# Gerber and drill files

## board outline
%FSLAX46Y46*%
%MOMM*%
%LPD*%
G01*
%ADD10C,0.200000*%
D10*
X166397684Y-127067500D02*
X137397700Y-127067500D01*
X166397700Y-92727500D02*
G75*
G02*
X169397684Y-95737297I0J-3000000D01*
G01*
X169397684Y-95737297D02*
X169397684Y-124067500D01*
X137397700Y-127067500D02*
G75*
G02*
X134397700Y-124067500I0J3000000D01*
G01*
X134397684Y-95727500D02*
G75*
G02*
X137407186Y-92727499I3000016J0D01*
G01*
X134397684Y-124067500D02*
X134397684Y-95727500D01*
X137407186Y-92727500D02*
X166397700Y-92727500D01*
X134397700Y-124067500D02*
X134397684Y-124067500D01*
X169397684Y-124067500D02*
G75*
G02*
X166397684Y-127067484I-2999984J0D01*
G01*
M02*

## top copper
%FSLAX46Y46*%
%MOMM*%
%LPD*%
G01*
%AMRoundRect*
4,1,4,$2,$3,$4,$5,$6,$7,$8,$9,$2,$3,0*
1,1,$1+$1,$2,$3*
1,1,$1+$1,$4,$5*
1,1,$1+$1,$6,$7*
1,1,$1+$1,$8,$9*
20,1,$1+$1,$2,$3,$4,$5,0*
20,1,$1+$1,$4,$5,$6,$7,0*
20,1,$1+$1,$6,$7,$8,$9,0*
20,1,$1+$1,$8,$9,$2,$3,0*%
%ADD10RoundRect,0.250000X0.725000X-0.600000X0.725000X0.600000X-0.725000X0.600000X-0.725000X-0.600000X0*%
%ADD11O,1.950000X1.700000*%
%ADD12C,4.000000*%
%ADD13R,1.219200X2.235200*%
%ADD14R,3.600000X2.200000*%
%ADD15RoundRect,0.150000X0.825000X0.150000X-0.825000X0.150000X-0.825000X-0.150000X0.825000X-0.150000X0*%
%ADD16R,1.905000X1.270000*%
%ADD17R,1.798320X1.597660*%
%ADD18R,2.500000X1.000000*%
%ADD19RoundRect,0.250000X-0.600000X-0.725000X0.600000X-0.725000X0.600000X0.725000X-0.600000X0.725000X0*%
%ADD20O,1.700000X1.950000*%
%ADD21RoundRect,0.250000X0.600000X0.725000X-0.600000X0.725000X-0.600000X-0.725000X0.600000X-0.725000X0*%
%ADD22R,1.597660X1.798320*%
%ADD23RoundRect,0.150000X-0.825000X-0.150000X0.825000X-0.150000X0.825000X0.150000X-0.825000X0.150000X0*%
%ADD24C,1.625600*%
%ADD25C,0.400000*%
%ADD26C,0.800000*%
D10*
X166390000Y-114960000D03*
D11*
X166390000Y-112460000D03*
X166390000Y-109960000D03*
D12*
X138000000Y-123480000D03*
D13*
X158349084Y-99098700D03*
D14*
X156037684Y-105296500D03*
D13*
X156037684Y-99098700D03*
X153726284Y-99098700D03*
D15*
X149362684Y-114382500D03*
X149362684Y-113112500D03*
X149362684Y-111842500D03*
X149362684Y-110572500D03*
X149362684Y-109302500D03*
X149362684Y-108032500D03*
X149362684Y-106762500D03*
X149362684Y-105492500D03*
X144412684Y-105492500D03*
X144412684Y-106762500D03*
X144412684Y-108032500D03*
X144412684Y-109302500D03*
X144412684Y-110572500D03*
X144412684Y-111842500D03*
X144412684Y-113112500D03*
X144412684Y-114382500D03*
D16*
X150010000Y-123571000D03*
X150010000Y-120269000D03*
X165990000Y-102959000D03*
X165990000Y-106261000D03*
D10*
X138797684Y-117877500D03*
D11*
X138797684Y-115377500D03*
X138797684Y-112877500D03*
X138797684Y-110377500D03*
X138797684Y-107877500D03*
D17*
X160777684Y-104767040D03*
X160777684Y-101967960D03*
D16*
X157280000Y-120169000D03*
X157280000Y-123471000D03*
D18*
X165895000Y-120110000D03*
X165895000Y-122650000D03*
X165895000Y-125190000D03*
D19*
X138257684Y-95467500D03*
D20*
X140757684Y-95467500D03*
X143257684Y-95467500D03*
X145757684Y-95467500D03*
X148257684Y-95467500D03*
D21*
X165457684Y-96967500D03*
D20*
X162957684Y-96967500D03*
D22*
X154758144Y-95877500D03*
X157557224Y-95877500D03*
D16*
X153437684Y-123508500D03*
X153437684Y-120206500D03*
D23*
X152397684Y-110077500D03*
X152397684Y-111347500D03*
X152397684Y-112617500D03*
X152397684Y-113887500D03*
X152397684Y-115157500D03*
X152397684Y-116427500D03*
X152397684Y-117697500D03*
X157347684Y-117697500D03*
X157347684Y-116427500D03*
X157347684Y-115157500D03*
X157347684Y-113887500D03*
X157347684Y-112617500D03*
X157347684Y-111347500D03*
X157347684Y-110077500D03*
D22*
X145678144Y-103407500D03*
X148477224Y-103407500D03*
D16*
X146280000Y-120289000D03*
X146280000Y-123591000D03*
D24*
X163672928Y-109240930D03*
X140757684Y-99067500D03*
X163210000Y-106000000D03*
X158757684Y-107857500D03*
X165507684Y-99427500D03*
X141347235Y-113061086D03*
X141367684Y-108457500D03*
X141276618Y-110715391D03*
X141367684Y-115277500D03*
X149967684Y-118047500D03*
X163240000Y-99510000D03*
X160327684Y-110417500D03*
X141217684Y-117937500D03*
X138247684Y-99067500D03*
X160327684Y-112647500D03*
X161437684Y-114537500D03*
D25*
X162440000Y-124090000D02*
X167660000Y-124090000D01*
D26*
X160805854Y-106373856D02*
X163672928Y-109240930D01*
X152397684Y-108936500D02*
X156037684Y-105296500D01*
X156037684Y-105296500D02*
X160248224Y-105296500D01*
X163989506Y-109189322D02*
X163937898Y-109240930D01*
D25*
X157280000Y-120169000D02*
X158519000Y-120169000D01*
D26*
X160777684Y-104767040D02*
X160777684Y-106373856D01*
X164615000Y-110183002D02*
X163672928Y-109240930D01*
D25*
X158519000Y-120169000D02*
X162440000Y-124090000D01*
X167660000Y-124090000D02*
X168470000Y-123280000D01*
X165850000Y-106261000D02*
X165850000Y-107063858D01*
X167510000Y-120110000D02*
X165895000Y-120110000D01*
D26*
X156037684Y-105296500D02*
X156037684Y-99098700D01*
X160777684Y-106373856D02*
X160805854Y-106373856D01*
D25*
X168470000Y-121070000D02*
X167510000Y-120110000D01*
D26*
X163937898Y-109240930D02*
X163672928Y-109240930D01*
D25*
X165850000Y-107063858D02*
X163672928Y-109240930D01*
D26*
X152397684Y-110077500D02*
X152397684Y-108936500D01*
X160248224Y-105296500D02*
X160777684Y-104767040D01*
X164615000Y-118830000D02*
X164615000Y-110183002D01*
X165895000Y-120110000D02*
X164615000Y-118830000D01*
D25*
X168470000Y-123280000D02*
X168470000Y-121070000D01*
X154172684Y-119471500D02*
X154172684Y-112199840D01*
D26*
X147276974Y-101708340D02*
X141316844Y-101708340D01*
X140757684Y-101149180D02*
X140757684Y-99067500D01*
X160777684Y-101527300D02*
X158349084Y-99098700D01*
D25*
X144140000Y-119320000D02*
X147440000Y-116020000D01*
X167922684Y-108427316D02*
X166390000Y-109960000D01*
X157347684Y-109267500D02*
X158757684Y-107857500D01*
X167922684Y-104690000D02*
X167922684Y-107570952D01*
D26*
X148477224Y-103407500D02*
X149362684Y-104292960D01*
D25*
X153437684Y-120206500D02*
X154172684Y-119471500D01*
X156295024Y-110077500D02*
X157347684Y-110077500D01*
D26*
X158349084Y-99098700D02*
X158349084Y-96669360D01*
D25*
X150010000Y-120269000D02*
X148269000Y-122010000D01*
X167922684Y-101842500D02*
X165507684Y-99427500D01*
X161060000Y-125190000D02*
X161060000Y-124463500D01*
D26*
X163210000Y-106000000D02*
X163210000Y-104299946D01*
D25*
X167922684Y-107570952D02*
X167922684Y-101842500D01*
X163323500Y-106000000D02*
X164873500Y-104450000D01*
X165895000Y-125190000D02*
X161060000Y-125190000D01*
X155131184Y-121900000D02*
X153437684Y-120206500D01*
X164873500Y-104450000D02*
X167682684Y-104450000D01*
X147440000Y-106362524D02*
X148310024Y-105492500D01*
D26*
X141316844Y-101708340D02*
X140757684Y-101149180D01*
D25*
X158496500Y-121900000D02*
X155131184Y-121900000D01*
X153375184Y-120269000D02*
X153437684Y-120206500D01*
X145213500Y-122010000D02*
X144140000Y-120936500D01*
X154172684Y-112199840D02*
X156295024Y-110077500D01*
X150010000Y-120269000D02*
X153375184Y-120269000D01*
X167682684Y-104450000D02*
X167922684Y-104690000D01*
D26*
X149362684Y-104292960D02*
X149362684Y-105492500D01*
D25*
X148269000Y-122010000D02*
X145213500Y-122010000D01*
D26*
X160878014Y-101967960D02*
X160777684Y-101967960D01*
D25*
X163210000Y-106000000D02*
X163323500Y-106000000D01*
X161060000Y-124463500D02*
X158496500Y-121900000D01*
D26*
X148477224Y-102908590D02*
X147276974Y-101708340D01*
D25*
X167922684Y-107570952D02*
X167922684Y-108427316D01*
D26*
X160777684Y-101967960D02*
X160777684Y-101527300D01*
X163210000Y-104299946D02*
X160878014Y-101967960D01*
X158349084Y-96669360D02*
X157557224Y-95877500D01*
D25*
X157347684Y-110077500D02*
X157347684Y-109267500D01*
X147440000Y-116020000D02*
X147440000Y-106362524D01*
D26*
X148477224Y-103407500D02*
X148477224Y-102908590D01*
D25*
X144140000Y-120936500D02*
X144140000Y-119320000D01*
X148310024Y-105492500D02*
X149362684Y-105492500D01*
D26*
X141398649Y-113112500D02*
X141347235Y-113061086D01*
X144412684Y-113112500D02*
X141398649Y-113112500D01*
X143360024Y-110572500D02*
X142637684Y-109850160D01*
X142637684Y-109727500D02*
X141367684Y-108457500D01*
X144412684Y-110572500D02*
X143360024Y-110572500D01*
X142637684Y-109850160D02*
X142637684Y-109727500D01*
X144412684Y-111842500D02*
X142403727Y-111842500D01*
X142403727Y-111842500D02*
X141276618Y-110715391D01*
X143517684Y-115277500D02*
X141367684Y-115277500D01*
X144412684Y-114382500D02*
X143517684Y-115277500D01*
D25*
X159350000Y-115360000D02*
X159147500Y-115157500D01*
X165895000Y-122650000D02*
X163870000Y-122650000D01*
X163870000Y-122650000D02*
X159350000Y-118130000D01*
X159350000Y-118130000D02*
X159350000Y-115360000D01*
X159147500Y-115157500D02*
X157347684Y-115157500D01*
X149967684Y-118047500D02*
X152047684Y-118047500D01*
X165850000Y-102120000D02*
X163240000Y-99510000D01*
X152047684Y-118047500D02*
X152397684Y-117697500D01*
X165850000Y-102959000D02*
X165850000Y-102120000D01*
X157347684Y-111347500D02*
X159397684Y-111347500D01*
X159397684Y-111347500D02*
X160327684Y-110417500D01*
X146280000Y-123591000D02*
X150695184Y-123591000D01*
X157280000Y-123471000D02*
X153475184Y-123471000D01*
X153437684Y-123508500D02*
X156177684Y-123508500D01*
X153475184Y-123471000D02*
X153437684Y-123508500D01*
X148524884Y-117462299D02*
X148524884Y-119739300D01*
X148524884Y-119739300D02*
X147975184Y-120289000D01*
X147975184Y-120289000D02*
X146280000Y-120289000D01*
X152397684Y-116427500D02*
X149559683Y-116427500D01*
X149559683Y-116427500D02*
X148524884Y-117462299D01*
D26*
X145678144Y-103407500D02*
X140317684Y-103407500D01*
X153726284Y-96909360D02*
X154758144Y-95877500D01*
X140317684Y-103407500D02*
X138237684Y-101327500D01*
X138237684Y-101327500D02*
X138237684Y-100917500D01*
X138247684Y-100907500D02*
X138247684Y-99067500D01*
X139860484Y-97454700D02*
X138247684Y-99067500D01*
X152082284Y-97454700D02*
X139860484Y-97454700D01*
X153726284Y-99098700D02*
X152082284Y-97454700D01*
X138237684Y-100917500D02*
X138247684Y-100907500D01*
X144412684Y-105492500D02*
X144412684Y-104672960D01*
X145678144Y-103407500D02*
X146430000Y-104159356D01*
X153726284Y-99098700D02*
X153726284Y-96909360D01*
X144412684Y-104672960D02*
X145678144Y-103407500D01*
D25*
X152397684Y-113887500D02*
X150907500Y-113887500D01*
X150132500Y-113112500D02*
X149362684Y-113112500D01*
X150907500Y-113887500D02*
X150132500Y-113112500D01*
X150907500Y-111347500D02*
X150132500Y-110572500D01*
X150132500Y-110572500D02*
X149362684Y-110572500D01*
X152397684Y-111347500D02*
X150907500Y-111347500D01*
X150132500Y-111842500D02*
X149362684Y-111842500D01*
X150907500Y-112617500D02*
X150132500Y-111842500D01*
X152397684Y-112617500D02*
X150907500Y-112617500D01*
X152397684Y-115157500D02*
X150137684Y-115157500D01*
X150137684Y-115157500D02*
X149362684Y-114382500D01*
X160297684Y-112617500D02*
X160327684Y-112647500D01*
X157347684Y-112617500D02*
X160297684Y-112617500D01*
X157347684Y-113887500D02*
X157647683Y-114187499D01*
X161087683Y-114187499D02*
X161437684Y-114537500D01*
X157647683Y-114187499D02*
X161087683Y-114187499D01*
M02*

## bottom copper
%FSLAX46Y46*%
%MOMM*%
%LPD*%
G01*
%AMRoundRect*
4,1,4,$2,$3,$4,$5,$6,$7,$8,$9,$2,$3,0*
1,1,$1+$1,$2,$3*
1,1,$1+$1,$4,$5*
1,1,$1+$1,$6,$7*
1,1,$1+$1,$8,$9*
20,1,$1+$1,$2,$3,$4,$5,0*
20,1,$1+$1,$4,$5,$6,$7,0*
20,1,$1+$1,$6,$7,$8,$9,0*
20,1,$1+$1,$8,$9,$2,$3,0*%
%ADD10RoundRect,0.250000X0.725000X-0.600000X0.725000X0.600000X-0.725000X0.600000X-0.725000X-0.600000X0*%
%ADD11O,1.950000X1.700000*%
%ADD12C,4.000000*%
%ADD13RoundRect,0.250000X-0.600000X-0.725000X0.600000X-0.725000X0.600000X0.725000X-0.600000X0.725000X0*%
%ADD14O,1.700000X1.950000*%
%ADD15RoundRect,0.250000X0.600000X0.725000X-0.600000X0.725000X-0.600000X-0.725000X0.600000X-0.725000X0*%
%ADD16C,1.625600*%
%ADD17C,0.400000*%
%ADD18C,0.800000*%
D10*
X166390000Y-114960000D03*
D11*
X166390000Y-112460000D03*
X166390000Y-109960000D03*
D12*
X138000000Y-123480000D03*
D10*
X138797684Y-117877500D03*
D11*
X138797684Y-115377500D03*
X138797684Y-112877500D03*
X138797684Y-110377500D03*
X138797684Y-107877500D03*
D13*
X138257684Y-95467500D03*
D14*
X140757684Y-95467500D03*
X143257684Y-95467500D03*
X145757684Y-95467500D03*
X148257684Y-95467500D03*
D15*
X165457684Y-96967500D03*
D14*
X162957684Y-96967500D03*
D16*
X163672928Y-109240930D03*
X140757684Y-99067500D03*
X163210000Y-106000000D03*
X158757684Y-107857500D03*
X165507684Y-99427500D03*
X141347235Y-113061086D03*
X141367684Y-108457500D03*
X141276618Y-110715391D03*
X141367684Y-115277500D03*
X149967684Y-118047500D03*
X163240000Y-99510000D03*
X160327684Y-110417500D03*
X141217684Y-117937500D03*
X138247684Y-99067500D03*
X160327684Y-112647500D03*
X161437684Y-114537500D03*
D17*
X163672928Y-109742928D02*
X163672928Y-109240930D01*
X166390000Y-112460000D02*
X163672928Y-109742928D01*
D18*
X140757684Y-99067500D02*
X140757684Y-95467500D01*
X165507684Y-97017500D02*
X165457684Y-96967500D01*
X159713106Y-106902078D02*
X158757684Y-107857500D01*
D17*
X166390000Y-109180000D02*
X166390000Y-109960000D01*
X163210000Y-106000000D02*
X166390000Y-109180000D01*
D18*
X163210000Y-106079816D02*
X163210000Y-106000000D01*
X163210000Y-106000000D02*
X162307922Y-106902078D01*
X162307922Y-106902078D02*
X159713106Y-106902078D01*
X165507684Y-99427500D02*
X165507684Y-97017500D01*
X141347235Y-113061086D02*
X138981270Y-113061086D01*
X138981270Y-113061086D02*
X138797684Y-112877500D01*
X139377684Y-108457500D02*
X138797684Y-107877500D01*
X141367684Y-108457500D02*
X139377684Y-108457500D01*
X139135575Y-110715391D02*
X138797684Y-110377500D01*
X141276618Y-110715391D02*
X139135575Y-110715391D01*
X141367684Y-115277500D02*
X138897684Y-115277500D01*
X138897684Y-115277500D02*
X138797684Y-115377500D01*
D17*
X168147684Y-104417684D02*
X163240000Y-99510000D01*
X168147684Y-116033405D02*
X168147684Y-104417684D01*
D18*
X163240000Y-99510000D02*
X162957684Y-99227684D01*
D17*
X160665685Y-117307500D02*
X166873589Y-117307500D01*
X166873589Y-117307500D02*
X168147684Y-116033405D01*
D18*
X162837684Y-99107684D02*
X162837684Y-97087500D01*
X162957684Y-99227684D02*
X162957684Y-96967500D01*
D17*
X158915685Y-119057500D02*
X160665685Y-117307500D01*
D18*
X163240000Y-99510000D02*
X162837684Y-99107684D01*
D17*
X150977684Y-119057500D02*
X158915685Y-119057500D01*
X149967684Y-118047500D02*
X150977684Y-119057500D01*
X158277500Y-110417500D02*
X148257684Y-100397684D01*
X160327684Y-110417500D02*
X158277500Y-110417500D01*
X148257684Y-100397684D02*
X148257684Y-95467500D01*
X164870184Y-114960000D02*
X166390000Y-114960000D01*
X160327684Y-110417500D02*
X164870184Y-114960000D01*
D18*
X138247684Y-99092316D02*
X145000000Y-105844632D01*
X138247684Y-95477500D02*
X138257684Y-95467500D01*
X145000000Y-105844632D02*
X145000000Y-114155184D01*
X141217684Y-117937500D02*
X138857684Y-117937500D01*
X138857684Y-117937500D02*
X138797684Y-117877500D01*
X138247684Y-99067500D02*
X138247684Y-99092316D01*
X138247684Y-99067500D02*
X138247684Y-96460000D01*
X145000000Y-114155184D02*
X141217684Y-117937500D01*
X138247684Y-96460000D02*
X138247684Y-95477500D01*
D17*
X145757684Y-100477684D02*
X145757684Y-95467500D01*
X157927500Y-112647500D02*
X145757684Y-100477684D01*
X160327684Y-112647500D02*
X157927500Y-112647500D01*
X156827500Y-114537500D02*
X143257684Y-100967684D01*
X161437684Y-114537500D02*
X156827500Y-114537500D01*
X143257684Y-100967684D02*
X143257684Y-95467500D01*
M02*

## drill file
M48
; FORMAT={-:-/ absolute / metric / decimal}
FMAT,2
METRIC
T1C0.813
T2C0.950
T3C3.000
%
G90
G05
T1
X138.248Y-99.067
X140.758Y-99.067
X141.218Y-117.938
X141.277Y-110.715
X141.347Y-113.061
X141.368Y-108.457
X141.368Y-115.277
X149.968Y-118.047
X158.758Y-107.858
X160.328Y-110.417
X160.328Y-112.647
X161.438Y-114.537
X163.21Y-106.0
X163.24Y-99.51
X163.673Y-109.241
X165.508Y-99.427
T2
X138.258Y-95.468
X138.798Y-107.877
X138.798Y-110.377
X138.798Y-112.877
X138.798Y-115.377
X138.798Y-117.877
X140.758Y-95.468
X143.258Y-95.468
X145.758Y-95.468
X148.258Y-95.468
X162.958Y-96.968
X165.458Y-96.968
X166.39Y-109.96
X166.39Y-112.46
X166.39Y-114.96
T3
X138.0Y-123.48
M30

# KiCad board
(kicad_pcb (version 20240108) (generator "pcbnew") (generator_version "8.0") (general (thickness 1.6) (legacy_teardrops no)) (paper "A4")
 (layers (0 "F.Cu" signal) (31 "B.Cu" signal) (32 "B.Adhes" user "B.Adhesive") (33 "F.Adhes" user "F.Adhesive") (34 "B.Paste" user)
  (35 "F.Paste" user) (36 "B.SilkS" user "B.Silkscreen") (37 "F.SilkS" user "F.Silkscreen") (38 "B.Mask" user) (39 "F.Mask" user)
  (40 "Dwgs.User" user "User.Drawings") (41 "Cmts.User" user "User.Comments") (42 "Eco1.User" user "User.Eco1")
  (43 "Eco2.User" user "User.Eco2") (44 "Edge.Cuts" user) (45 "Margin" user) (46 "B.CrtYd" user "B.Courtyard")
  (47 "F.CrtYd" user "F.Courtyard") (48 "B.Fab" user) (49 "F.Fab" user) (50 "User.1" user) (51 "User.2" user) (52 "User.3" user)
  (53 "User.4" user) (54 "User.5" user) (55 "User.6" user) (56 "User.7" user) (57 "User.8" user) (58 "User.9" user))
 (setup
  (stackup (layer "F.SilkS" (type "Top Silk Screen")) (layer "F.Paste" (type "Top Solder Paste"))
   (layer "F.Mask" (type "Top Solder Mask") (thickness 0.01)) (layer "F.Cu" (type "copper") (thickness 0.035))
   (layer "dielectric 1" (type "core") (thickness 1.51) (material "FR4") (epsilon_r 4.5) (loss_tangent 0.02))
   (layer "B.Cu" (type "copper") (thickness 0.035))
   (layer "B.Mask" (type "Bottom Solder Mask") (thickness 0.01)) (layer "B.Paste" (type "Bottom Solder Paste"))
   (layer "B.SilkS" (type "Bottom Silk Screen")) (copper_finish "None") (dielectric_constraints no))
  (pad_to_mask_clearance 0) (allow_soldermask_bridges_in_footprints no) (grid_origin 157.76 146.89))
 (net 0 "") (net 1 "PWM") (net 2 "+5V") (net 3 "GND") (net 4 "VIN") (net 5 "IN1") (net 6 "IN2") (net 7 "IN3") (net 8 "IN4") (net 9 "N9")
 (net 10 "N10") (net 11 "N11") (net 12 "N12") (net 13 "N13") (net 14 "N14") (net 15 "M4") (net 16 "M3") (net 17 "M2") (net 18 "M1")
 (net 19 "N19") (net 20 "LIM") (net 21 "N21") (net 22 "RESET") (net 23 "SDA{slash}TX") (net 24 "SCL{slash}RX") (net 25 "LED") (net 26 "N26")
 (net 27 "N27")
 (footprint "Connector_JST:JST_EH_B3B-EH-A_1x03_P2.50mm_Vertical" (layer "F.Cu") (at 166.39 114.96 90)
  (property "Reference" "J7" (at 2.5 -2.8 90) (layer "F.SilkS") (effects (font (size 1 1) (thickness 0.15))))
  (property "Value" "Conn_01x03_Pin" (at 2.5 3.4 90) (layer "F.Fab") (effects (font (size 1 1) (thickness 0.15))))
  (pad "1" thru_hole roundrect (at 0 0 90) (size 1.7 1.95) (drill 0.95) (layers "*.Cu" "*.Mask") (remove_unused_layers no)
   (roundrect_rratio 0.147059) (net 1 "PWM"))
  (pad "2" thru_hole oval (at 2.5 0 90) (size 1.7 1.95) (drill 0.95) (layers "*.Cu" "*.Mask") (remove_unused_layers no) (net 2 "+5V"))
  (pad "3" thru_hole oval (at 5 0 90) (size 1.7 1.95) (drill 0.95) (layers "*.Cu" "*.Mask") (remove_unused_layers no) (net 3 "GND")))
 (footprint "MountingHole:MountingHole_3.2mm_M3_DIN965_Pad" (layer "F.Cu") (at 138 123.48)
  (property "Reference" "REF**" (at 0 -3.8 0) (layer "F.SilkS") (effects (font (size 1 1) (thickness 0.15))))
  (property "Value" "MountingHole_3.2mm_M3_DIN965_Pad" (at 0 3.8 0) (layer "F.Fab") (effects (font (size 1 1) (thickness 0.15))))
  (pad "1" thru_hole circle (at 0 0) (size 4 4) (drill 3) (layers "*.Cu" "*.Mask") (remove_unused_layers no)))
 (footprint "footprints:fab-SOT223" (layer "F.Cu") (at 156.037684 102.1975 180)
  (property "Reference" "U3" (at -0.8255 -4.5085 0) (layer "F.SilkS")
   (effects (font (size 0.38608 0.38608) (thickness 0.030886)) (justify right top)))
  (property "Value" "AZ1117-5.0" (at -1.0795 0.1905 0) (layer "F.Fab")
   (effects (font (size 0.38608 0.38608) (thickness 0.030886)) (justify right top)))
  (pad "1" smd rect (at -2.3114 3.0988 180) (size 1.2192 2.2352) (layers "F.Cu" "F.Paste" "F.Mask") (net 3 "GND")
   (solder_mask_margin 0.1016))
  (pad "2" smd rect (at 0 -3.099 180) (size 3.6 2.2) (layers "F.Cu" "F.Paste" "F.Mask") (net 2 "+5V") (solder_mask_margin 0.1016))
  (pad "2" smd rect (at 0 3.0988 180) (size 1.2192 2.2352) (layers "F.Cu" "F.Paste" "F.Mask") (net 2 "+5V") (solder_mask_margin 0.1016))
  (pad "3" smd rect (at 2.3114 3.0988 180) (size 1.2192 2.2352) (layers "F.Cu" "F.Paste" "F.Mask") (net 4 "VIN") (solder_mask_margin 0.1016)))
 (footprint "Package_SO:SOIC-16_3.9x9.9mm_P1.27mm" (layer "F.Cu") (at 146.887684 109.9375 180)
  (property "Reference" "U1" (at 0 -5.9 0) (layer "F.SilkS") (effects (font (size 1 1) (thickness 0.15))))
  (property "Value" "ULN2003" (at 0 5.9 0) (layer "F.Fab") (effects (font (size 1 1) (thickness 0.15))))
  (pad "1" smd roundrect (at -2.475 -4.445 180) (size 1.95 0.6) (layers "F.Cu" "F.Paste" "F.Mask") (roundrect_rratio 0.25) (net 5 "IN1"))
  (pad "2" smd roundrect (at -2.475 -3.175 180) (size 1.95 0.6) (layers "F.Cu" "F.Paste" "F.Mask") (roundrect_rratio 0.25) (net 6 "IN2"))
  (pad "3" smd roundrect (at -2.475 -1.905 180) (size 1.95 0.6) (layers "F.Cu" "F.Paste" "F.Mask") (roundrect_rratio 0.25) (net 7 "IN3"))
  (pad "4" smd roundrect (at -2.475 -0.635 180) (size 1.95 0.6) (layers "F.Cu" "F.Paste" "F.Mask") (roundrect_rratio 0.25) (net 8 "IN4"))
  (pad "5" smd roundrect (at -2.475 0.635 180) (size 1.95 0.6) (layers "F.Cu" "F.Paste" "F.Mask") (roundrect_rratio 0.25) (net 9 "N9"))
  (pad "6" smd roundrect (at -2.475 1.905 180) (size 1.95 0.6) (layers "F.Cu" "F.Paste" "F.Mask") (roundrect_rratio 0.25) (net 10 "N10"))
  (pad "7" smd roundrect (at -2.475 3.175 180) (size 1.95 0.6) (layers "F.Cu" "F.Paste" "F.Mask") (roundrect_rratio 0.25) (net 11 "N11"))
  (pad "8" smd roundrect (at -2.475 4.445 180) (size 1.95 0.6) (layers "F.Cu" "F.Paste" "F.Mask") (roundrect_rratio 0.25) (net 3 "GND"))
  (pad "9" smd roundrect (at 2.475 4.445 180) (size 1.95 0.6) (layers "F.Cu" "F.Paste" "F.Mask") (roundrect_rratio 0.25) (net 4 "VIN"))
  (pad "10" smd roundrect (at 2.475 3.175 180) (size 1.95 0.6) (layers "F.Cu" "F.Paste" "F.Mask") (roundrect_rratio 0.25) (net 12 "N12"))
  (pad "11" smd roundrect (at 2.475 1.905 180) (size 1.95 0.6) (layers "F.Cu" "F.Paste" "F.Mask") (roundrect_rratio 0.25) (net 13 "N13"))
  (pad "12" smd roundrect (at 2.475 0.635 180) (size 1.95 0.6) (layers "F.Cu" "F.Paste" "F.Mask") (roundrect_rratio 0.25) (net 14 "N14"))
  (pad "13" smd roundrect (at 2.475 -0.635 180) (size 1.95 0.6) (layers "F.Cu" "F.Paste" "F.Mask") (roundrect_rratio 0.25) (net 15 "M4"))
  (pad "14" smd roundrect (at 2.475 -1.905 180) (size 1.95 0.6) (layers "F.Cu" "F.Paste" "F.Mask") (roundrect_rratio 0.25) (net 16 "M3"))
  (pad "15" smd roundrect (at 2.475 -3.175 180) (size 1.95 0.6) (layers "F.Cu" "F.Paste" "F.Mask") (roundrect_rratio 0.25) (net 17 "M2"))
  (pad "16" smd roundrect (at 2.475 -4.445 180) (size 1.95 0.6) (layers "F.Cu" "F.Paste" "F.Mask") (roundrect_rratio 0.25) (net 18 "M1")))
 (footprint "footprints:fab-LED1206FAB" (layer "F.Cu") (at 150.01 121.92 90)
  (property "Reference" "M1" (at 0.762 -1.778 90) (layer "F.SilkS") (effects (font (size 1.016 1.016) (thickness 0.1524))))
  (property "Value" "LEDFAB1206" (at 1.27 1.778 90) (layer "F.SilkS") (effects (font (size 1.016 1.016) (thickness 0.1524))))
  (pad "1" smd rect (at -1.651 0 90) (size 1.27 1.905) (layers "F.Cu" "F.Paste" "F.Mask") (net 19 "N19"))
  (pad "2" smd rect (at 1.651 0 90) (size 1.27 1.905) (layers "F.Cu" "F.Paste" "F.Mask") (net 3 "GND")))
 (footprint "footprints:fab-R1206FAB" (layer "F.Cu") (at 165.99 104.61 -90)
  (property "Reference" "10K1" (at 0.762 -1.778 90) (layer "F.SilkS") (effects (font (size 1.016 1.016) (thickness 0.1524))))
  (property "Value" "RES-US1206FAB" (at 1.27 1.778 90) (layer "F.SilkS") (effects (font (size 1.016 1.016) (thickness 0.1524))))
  (pad "1" smd rect (at -1.651 0 270) (size 1.27 1.905) (layers "F.Cu" "F.Paste" "F.Mask") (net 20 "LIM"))
  (pad "2" smd rect (at 1.651 0 270) (size 1.27 1.905) (layers "F.Cu" "F.Paste" "F.Mask") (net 2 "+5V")))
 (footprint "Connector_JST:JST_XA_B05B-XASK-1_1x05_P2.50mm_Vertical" (layer "F.Cu") (at 138.797684 117.8775 90)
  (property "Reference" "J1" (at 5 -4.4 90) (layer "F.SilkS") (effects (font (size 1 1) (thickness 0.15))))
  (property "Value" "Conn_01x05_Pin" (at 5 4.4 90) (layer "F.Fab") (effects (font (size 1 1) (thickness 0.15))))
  (pad "1" thru_hole roundrect (at 0 0 90) (size 1.7 1.95) (drill 0.95) (layers "*.Cu" "*.Mask") (remove_unused_layers no)
   (roundrect_rratio 0.147059) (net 4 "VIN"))
  (pad "2" thru_hole oval (at 2.5 0 90) (size 1.7 1.95) (drill 0.95) (layers "*.Cu" "*.Mask") (remove_unused_layers no) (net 18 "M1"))
  (pad "3" thru_hole oval (at 5 0 90) (size 1.7 1.95) (drill 0.95) (layers "*.Cu" "*.Mask") (remove_unused_layers no) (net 17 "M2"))
  (pad "4" thru_hole oval (at 7.5 0 90) (size 1.7 1.95) (drill 0.95) (layers "*.Cu" "*.Mask") (remove_unused_layers no) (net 16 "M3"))
  (pad "5" thru_hole oval (at 10 0 90) (size 1.7 1.95) (drill 0.95) (layers "*.Cu" "*.Mask") (remove_unused_layers no) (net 15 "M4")))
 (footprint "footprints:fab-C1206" (layer "F.Cu") (at 160.777684 103.3675 90)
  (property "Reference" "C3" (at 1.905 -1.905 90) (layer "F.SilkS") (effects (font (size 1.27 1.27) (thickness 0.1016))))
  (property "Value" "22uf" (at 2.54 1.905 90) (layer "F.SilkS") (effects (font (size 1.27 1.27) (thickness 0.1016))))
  (pad "1" smd rect (at -1.39954 0 90) (size 1.59766 1.79832) (layers "F.Cu" "F.Paste" "F.Mask") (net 2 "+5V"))
  (pad "2" smd rect (at 1.39954 0 90) (size 1.59766 1.79832) (layers "F.Cu" "F.Paste" "F.Mask") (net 3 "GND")))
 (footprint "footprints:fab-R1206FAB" (layer "F.Cu") (at 157.28 121.82 -90)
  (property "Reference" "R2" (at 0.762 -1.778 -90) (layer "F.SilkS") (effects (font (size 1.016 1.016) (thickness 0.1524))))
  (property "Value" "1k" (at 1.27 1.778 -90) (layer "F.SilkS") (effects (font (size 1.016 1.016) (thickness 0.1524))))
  (pad "1" smd rect (at -1.651 0 270) (size 1.27 1.905) (layers "F.Cu" "F.Paste" "F.Mask") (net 2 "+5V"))
  (pad "2" smd rect (at 1.651 0 270) (size 1.27 1.905) (layers "F.Cu" "F.Paste" "F.Mask") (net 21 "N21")))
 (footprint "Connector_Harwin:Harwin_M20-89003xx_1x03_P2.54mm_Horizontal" (layer "F.Cu") (at 171.42 122.65)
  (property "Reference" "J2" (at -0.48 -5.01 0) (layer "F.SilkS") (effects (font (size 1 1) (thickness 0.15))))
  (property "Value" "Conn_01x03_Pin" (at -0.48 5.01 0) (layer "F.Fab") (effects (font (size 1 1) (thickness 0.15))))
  (pad "" smd rect (at 3.895 -2.54) (size 6 0.76) (layers "F.SilkS"))
  (pad "1" smd rect (at -5.525 -2.54) (size 2.5 1) (layers "F.Cu" "F.Paste" "F.Mask") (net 2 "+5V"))
  (pad "2" smd rect (at -5.525 0) (size 2.5 1) (layers "F.Cu" "F.Paste" "F.Mask") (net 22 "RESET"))
  (pad "3" smd rect (at -5.525 2.54) (size 2.5 1) (layers "F.Cu" "F.Paste" "F.Mask") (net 3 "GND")))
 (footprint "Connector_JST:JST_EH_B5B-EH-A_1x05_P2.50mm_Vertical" (layer "F.Cu") (at 138.257684 95.4675)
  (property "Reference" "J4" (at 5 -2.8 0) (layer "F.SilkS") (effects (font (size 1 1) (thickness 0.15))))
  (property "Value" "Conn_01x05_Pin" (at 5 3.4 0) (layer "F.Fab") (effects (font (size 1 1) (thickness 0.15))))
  (pad "1" thru_hole roundrect (at 0 0) (size 1.7 1.95) (drill 0.95) (layers "*.Cu" "*.Mask") (remove_unused_layers no)
   (roundrect_rratio 0.147059) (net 4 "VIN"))
  (pad "2" thru_hole oval (at 2.5 0) (size 1.7 1.95) (drill 0.95) (layers "*.Cu" "*.Mask") (remove_unused_layers no) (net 3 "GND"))
  (pad "3" thru_hole oval (at 5 0) (size 1.7 1.95) (drill 0.95) (layers "*.Cu" "*.Mask") (remove_unused_layers no) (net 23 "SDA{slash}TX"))
  (pad "4" thru_hole oval (at 7.5 0) (size 1.7 1.95) (drill 0.95) (layers "*.Cu" "*.Mask") (remove_unused_layers no) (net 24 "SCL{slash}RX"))
  (pad "5" thru_hole oval (at 10 0) (size 1.7 1.95) (drill 0.95) (layers "*.Cu" "*.Mask") (remove_unused_layers no) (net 1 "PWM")))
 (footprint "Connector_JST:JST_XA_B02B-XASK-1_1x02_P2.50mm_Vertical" (layer "F.Cu") (at 165.457684 96.9675 180)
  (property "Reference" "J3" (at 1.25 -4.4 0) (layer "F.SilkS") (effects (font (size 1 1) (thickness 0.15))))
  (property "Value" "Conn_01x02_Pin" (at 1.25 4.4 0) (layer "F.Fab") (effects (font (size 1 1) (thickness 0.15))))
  (pad "1" thru_hole roundrect (at 0 0 180) (size 1.7 1.95) (drill 0.95) (layers "*.Cu" "*.Mask") (remove_unused_layers no)
   (roundrect_rratio 0.147059) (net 3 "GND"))
  (pad "2" thru_hole oval (at 2.5 0 180) (size 1.7 1.95) (drill 0.95) (layers "*.Cu" "*.Mask") (remove_unused_layers no) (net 20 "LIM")))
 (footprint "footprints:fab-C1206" (layer "F.Cu") (at 156.157684 95.8775)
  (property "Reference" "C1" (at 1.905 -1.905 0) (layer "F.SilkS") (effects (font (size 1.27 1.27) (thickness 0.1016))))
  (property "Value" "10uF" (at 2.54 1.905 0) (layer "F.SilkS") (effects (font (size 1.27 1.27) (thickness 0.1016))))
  (pad "1" smd rect (at -1.39954 0) (size 1.59766 1.79832) (layers "F.Cu" "F.Paste" "F.Mask") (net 4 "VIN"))
  (pad "2" smd rect (at 1.39954 0) (size 1.59766 1.79832) (layers "F.Cu" "F.Paste" "F.Mask") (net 3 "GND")))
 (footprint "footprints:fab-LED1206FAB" (layer "F.Cu") (at 153.437684 121.8575 90)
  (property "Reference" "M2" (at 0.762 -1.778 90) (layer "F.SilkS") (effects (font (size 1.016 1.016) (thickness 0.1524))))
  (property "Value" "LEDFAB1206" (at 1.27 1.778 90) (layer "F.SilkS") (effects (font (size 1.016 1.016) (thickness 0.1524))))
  (pad "1" smd rect (at -1.651 0 90) (size 1.27 1.905) (layers "F.Cu" "F.Paste" "F.Mask") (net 21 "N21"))
  (pad "2" smd rect (at 1.651 0 90) (size 1.27 1.905) (layers "F.Cu" "F.Paste" "F.Mask") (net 3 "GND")))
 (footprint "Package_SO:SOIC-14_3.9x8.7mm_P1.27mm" (layer "F.Cu") (at 154.872684 113.8875)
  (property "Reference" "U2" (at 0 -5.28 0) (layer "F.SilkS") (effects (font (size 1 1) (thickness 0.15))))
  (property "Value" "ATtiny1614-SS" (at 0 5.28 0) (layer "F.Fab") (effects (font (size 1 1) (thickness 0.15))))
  (pad "1" smd roundrect (at -2.475 -3.81) (size 1.95 0.6) (layers "F.Cu" "F.Paste" "F.Mask") (roundrect_rratio 0.25) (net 2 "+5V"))
  (pad "2" smd roundrect (at -2.475 -2.54) (size 1.95 0.6) (layers "F.Cu" "F.Paste" "F.Mask") (roundrect_rratio 0.25) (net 8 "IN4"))
  (pad "3" smd roundrect (at -2.475 -1.27) (size 1.95 0.6) (layers "F.Cu" "F.Paste" "F.Mask") (roundrect_rratio 0.25) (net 7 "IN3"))
  (pad "4" smd roundrect (at -2.475 0) (size 1.95 0.6) (layers "F.Cu" "F.Paste" "F.Mask") (roundrect_rratio 0.25) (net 6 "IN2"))
  (pad "5" smd roundrect (at -2.475 1.27) (size 1.95 0.6) (layers "F.Cu" "F.Paste" "F.Mask") (roundrect_rratio 0.25) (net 5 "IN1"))
  (pad "6" smd roundrect (at -2.475 2.54) (size 1.95 0.6) (layers "F.Cu" "F.Paste" "F.Mask") (roundrect_rratio 0.25) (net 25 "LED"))
  (pad "7" smd roundrect (at -2.475 3.81) (size 1.95 0.6) (layers "F.Cu" "F.Paste" "F.Mask") (roundrect_rratio 0.25) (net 20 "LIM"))
  (pad "8" smd roundrect (at 2.475 3.81) (size 1.95 0.6) (layers "F.Cu" "F.Paste" "F.Mask") (roundrect_rratio 0.25) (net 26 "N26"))
  (pad "9" smd roundrect (at 2.475 2.54) (size 1.95 0.6) (layers "F.Cu" "F.Paste" "F.Mask") (roundrect_rratio 0.25) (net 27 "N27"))
  (pad "10" smd roundrect (at 2.475 1.27) (size 1.95 0.6) (layers "F.Cu" "F.Paste" "F.Mask") (roundrect_rratio 0.25) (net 22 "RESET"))
  (pad "11" smd roundrect (at 2.475 0) (size 1.95 0.6) (layers "F.Cu" "F.Paste" "F.Mask") (roundrect_rratio 0.25) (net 23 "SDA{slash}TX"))
  (pad "12" smd roundrect (at 2.475 -1.27) (size 1.95 0.6) (layers "F.Cu" "F.Paste" "F.Mask") (roundrect_rratio 0.25)
   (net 24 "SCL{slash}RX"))
  (pad "13" smd roundrect (at 2.475 -2.54) (size 1.95 0.6) (layers "F.Cu" "F.Paste" "F.Mask") (roundrect_rratio 0.25) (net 1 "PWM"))
  (pad "14" smd roundrect (at 2.475 -3.81) (size 1.95 0.6) (layers "F.Cu" "F.Paste" "F.Mask") (roundrect_rratio 0.25) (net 3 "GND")))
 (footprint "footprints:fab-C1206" (layer "F.Cu") (at 147.077684 103.4075)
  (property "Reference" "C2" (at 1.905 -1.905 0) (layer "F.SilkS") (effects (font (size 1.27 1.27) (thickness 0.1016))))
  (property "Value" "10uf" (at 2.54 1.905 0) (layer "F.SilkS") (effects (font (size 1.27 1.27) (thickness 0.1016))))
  (pad "1" smd rect (at -1.39954 0) (size 1.59766 1.79832) (layers "F.Cu" "F.Paste" "F.Mask") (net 4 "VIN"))
  (pad "2" smd rect (at 1.39954 0) (size 1.59766 1.79832) (layers "F.Cu" "F.Paste" "F.Mask") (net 3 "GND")))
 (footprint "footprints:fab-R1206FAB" (layer "F.Cu") (at 146.28 121.94 -90)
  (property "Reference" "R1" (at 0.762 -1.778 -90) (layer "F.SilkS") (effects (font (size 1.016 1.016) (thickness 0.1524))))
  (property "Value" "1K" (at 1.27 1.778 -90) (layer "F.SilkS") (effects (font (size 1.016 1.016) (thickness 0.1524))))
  (pad "1" smd rect (at -1.651 0 270) (size 1.27 1.905) (layers "F.Cu" "F.Paste" "F.Mask") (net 25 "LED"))
  (pad "2" smd rect (at 1.651 0 270) (size 1.27 1.905) (layers "F.Cu" "F.Paste" "F.Mask") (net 19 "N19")))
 (gr_line (start 166.397684 127.0675) (end 137.3977 127.0675) (stroke (width 0.2) (type default)) (layer "Edge.Cuts"))
 (gr_arc (start 166.3977 92.7275) (mid 168.519006 93.606178) (end 169.397684 95.737297) (stroke (width 0.2) (type default))
  (layer "Edge.Cuts"))
 (gr_line (start 169.397684 95.737297) (end 169.397684 124.0675) (stroke (width 0.2) (type default)) (layer "Edge.Cuts"))
 (gr_arc (start 137.3977 127.0675) (mid 135.276366 126.188818) (end 134.3977 124.0675) (stroke (width 0.2) (type default))
  (layer "Edge.Cuts"))
 (gr_arc (start 134.397684 95.7275) (mid 135.276366 93.606182) (end 137.407186 92.7275) (stroke (width 0.2) (type default))
  (layer "Edge.Cuts"))
 (gr_line (start 134.397684 124.0675) (end 134.397684 95.7275) (stroke (width 0.2) (type default)) (layer "Edge.Cuts"))
 (gr_line (start 137.407186 92.7275) (end 166.3977 92.7275) (stroke (width 0.2) (type default)) (layer "Edge.Cuts"))
 (gr_line (start 134.3977 124.0675) (end 134.397684 124.0675) (stroke (width 0.2) (type default)) (layer "Edge.Cuts"))
 (gr_arc (start 169.397684 124.0675) (mid 168.519006 126.188822) (end 166.397684 127.0675) (stroke (width 0.2) (type default))
  (layer "Edge.Cuts"))
 (segment (start 162.44 124.09) (end 167.66 124.09) (width 0.4) (layer "F.Cu") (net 2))
 (segment (start 160.805854 106.373856) (end 163.672928 109.24093) (width 0.8) (layer "F.Cu") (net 2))
 (segment (start 152.397684 108.9365) (end 156.037684 105.2965) (width 0.8) (layer "F.Cu") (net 2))
 (segment (start 156.037684 105.2965) (end 160.248224 105.2965) (width 0.8) (layer "F.Cu") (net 2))
 (segment (start 163.989506 109.189322) (end 163.937898 109.24093) (width 0.8) (layer "F.Cu") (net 2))
 (segment (start 157.28 120.169) (end 158.519 120.169) (width 0.4) (layer "F.Cu") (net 2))
 (segment (start 160.777684 104.76704) (end 160.777684 106.373856) (width 0.8) (layer "F.Cu") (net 2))
 (segment (start 164.615 110.183002) (end 163.672928 109.24093) (width 0.8) (layer "F.Cu") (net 2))
 (segment (start 158.519 120.169) (end 162.44 124.09) (width 0.4) (layer "F.Cu") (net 2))
 (segment (start 167.66 124.09) (end 168.47 123.28) (width 0.4) (layer "F.Cu") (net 2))
 (segment (start 165.85 106.261) (end 165.85 107.063858) (width 0.4) (layer "F.Cu") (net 2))
 (segment (start 167.51 120.11) (end 165.895 120.11) (width 0.4) (layer "F.Cu") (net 2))
 (segment (start 156.037684 105.2965) (end 156.037684 99.0987) (width 0.8) (layer "F.Cu") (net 2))
 (segment (start 160.777684 106.373856) (end 160.805854 106.373856) (width 0.8) (layer "F.Cu") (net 2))
 (segment (start 168.47 121.07) (end 167.51 120.11) (width 0.4) (layer "F.Cu") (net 2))
 (segment (start 163.937898 109.24093) (end 163.672928 109.24093) (width 0.8) (layer "F.Cu") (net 2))
 (segment (start 165.85 107.063858) (end 163.672928 109.24093) (width 0.4) (layer "F.Cu") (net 2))
 (segment (start 152.397684 110.0775) (end 152.397684 108.9365) (width 0.8) (layer "F.Cu") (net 2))
 (segment (start 160.248224 105.2965) (end 160.777684 104.76704) (width 0.8) (layer "F.Cu") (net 2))
 (segment (start 164.615 118.83) (end 164.615 110.183002) (width 0.8) (layer "F.Cu") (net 2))
 (segment (start 165.895 120.11) (end 164.615 118.83) (width 0.8) (layer "F.Cu") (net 2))
 (segment (start 168.47 123.28) (end 168.47 121.07) (width 0.4) (layer "F.Cu") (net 2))
 (via (at 163.672928 109.24093) (size 1.6256) (drill 0.8128) (layers "F.Cu" "B.Cu") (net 2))
 (segment (start 163.672928 109.742928) (end 163.672928 109.24093) (width 0.4) (layer "B.Cu") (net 2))
 (segment (start 166.39 112.46) (end 163.672928 109.742928) (width 0.4) (layer "B.Cu") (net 2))
 (segment (start 154.172684 119.4715) (end 154.172684 112.19984) (width 0.4) (layer "F.Cu") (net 3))
 (segment (start 147.276974 101.70834) (end 141.316844 101.70834) (width 0.8) (layer "F.Cu") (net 3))
 (segment (start 140.757684 101.14918) (end 140.757684 99.0675) (width 0.8) (layer "F.Cu") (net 3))
 (segment (start 160.777684 101.5273) (end 158.349084 99.0987) (width 0.8) (layer "F.Cu") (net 3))
 (segment (start 144.14 119.32) (end 147.44 116.02) (width 0.4) (layer "F.Cu") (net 3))
 (segment (start 167.922684 108.427316) (end 166.39 109.96) (width 0.4) (layer "F.Cu") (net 3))
 (segment (start 157.347684 109.2675) (end 158.757684 107.8575) (width 0.4) (layer "F.Cu") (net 3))
 (segment (start 167.922684 104.69) (end 167.922684 107.570952) (width 0.4) (layer "F.Cu") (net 3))
 (segment (start 148.477224 103.4075) (end 149.362684 104.29296) (width 0.8) (layer "F.Cu") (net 3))
 (segment (start 153.437684 120.2065) (end 154.172684 119.4715) (width 0.4) (layer "F.Cu") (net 3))
 (segment (start 156.295024 110.0775) (end 157.347684 110.0775) (width 0.4) (layer "F.Cu") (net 3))
 (segment (start 158.349084 99.0987) (end 158.349084 96.66936) (width 0.8) (layer "F.Cu") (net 3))
 (segment (start 150.01 120.269) (end 148.269 122.01) (width 0.4) (layer "F.Cu") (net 3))
 (segment (start 167.922684 101.8425) (end 165.507684 99.4275) (width 0.4) (layer "F.Cu") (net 3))
 (segment (start 161.06 125.19) (end 161.06 124.4635) (width 0.4) (layer "F.Cu") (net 3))
 (segment (start 163.21 106) (end 163.21 104.299946) (width 0.8) (layer "F.Cu") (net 3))
 (segment (start 167.922684 107.570952) (end 167.922684 101.8425) (width 0.4) (layer "F.Cu") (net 3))
 (segment (start 163.3235 106) (end 164.8735 104.45) (width 0.4) (layer "F.Cu") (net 3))
 (segment (start 165.895 125.19) (end 161.06 125.19) (width 0.4) (layer "F.Cu") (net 3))
 (segment (start 155.131184 121.9) (end 153.437684 120.2065) (width 0.4) (layer "F.Cu") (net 3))
 (segment (start 164.8735 104.45) (end 167.682684 104.45) (width 0.4) (layer "F.Cu") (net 3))
 (segment (start 147.44 106.362524) (end 148.310024 105.4925) (width 0.4) (layer "F.Cu") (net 3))
 (segment (start 141.316844 101.70834) (end 140.757684 101.14918) (width 0.8) (layer "F.Cu") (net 3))
 (segment (start 158.4965 121.9) (end 155.131184 121.9) (width 0.4) (layer "F.Cu") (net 3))
 (segment (start 153.375184 120.269) (end 153.437684 120.2065) (width 0.4) (layer "F.Cu") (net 3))
 (segment (start 145.2135 122.01) (end 144.14 120.9365) (width 0.4) (layer "F.Cu") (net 3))
 (segment (start 154.172684 112.19984) (end 156.295024 110.0775) (width 0.4) (layer "F.Cu") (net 3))
 (segment (start 150.01 120.269) (end 153.375184 120.269) (width 0.4) (layer "F.Cu") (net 3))
 (segment (start 167.682684 104.45) (end 167.922684 104.69) (width 0.4) (layer "F.Cu") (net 3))
 (segment (start 149.362684 104.29296) (end 149.362684 105.4925) (width 0.8) (layer "F.Cu") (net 3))
 (segment (start 148.269 122.01) (end 145.2135 122.01) (width 0.4) (layer "F.Cu") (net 3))
 (segment (start 160.878014 101.96796) (end 160.777684 101.96796) (width 0.8) (layer "F.Cu") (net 3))
 (segment (start 163.21 106) (end 163.3235 106) (width 0.4) (layer "F.Cu") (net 3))
 (segment (start 161.06 124.4635) (end 158.4965 121.9) (width 0.4) (layer "F.Cu") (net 3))
 (segment (start 148.477224 102.90859) (end 147.276974 101.70834) (width 0.8) (layer "F.Cu") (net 3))
 (segment (start 167.922684 107.570952) (end 167.922684 108.427316) (width 0.4) (layer "F.Cu") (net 3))
 (segment (start 160.777684 101.96796) (end 160.777684 101.5273) (width 0.8) (layer "F.Cu") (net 3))
 (segment (start 163.21 104.299946) (end 160.878014 101.96796) (width 0.8) (layer "F.Cu") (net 3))
 (segment (start 158.349084 96.66936) (end 157.557224 95.8775) (width 0.8) (layer "F.Cu") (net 3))
 (segment (start 157.347684 110.0775) (end 157.347684 109.2675) (width 0.4) (layer "F.Cu") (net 3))
 (segment (start 147.44 116.02) (end 147.44 106.362524) (width 0.4) (layer "F.Cu") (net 3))
 (segment (start 148.477224 103.4075) (end 148.477224 102.90859) (width 0.8) (layer "F.Cu") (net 3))
 (segment (start 144.14 120.9365) (end 144.14 119.32) (width 0.4) (layer "F.Cu") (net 3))
 (segment (start 148.310024 105.4925) (end 149.362684 105.4925) (width 0.4) (layer "F.Cu") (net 3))
 (via (at 140.757684 99.0675) (size 1.6256) (drill 0.8128) (layers "F.Cu" "B.Cu") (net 3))
 (via (at 163.21 106) (size 1.6256) (drill 0.8128) (layers "F.Cu" "B.Cu") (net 3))
 (via (at 158.757684 107.8575) (size 1.6256) (drill 0.8128) (layers "F.Cu" "B.Cu") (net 3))
 (via (at 165.507684 99.4275) (size 1.6256) (drill 0.8128) (layers "F.Cu" "B.Cu") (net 3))
 (segment (start 140.757684 99.0675) (end 140.757684 95.4675) (width 0.8) (layer "B.Cu") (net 3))
 (segment (start 165.507684 97.0175) (end 165.457684 96.9675) (width 0.8) (layer "B.Cu") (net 3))
 (segment (start 159.713106 106.902078) (end 158.757684 107.8575) (width 0.8) (layer "B.Cu") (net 3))
 (segment (start 166.39 109.18) (end 166.39 109.96) (width 0.4) (layer "B.Cu") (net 3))
 (segment (start 163.21 106) (end 166.39 109.18) (width 0.4) (layer "B.Cu") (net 3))
 (segment (start 163.21 106.079816) (end 163.21 106) (width 0.8) (layer "B.Cu") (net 3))
 (segment (start 163.21 106) (end 162.307922 106.902078) (width 0.8) (layer "B.Cu") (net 3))
 (segment (start 162.307922 106.902078) (end 159.713106 106.902078) (width 0.8) (layer "B.Cu") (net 3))
 (segment (start 165.507684 99.4275) (end 165.507684 97.0175) (width 0.8) (layer "B.Cu") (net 3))
 (segment (start 141.398649 113.1125) (end 141.347235 113.061086) (width 0.8) (layer "F.Cu") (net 17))
 (segment (start 144.412684 113.1125) (end 141.398649 113.1125) (width 0.8) (layer "F.Cu") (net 17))
 (via (at 141.347235 113.061086) (size 1.6256) (drill 0.8128) (layers "F.Cu" "B.Cu") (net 17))
 (segment (start 141.347235 113.061086) (end 138.98127 113.061086) (width 0.8) (layer "B.Cu") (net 17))
 (segment (start 138.98127 113.061086) (end 138.797684 112.8775) (width 0.8) (layer "B.Cu") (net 17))
 (segment (start 143.360024 110.5725) (end 142.637684 109.85016) (width 0.8) (layer "F.Cu") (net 15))
 (segment (start 142.637684 109.7275) (end 141.367684 108.4575) (width 0.8) (layer "F.Cu") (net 15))
 (segment (start 144.412684 110.5725) (end 143.360024 110.5725) (width 0.8) (layer "F.Cu") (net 15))
 (segment (start 142.637684 109.85016) (end 142.637684 109.7275) (width 0.8) (layer "F.Cu") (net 15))
 (via (at 141.367684 108.4575) (size 1.6256) (drill 0.8128) (layers "F.Cu" "B.Cu") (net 15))
 (segment (start 139.377684 108.4575) (end 138.797684 107.8775) (width 0.8) (layer "B.Cu") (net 15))
 (segment (start 141.367684 108.4575) (end 139.377684 108.4575) (width 0.8) (layer "B.Cu") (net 15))
 (segment (start 144.412684 111.8425) (end 142.403727 111.8425) (width 0.8) (layer "F.Cu") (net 16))
 (segment (start 142.403727 111.8425) (end 141.276618 110.715391) (width 0.8) (layer "F.Cu") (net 16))
 (via (at 141.276618 110.715391) (size 1.6256) (drill 0.8128) (layers "F.Cu" "B.Cu") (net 16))
 (segment (start 139.135575 110.715391) (end 138.797684 110.3775) (width 0.8) (layer "B.Cu") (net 16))
 (segment (start 141.276618 110.715391) (end 139.135575 110.715391) (width 0.8) (layer "B.Cu") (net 16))
 (segment (start 143.517684 115.2775) (end 141.367684 115.2775) (width 0.8) (layer "F.Cu") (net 18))
 (segment (start 144.412684 114.3825) (end 143.517684 115.2775) (width 0.8) (layer "F.Cu") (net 18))
 (via (at 141.367684 115.2775) (size 1.6256) (drill 0.8128) (layers "F.Cu" "B.Cu") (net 18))
 (segment (start 141.367684 115.2775) (end 138.897684 115.2775) (width 0.8) (layer "B.Cu") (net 18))
 (segment (start 138.897684 115.2775) (end 138.797684 115.3775) (width 0.8) (layer "B.Cu") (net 18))
 (segment (start 159.35 115.36) (end 159.1475 115.1575) (width 0.4) (layer "F.Cu") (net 22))
 (segment (start 165.895 122.65) (end 163.87 122.65) (width 0.4) (layer "F.Cu") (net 22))
 (segment (start 163.87 122.65) (end 159.35 118.13) (width 0.4) (layer "F.Cu") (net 22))
 (segment (start 159.35 118.13) (end 159.35 115.36) (width 0.4) (layer "F.Cu") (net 22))
 (segment (start 159.1475 115.1575) (end 157.347684 115.1575) (width 0.4) (layer "F.Cu") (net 22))
 (segment (start 149.967684 118.0475) (end 152.047684 118.0475) (width 0.4) (layer "F.Cu") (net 20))
 (segment (start 165.85 102.12) (end 163.24 99.51) (width 0.4) (layer "F.Cu") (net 20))
 (segment (start 152.047684 118.0475) (end 152.397684 117.6975) (width 0.4) (layer "F.Cu") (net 20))
 (segment (start 165.85 102.959) (end 165.85 102.12) (width 0.4) (layer "F.Cu") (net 20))
 (via (at 149.967684 118.0475) (size 1.6256) (drill 0.8128) (layers "F.Cu" "B.Cu") (free yes) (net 20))
 (via (at 163.24 99.51) (size 1.6256) (drill 0.8128) (layers "F.Cu" "B.Cu") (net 20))
 (segment (start 168.147684 104.417684) (end 163.24 99.51) (width 0.4) (layer "B.Cu") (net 20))
 (segment (start 168.147684 116.033405) (end 168.147684 104.417684) (width 0.4) (layer "B.Cu") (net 20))
 (segment (start 163.24 99.51) (end 162.957684 99.227684) (width 0.8) (layer "B.Cu") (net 20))
 (segment (start 160.665685 117.3075) (end 166.873589 117.3075) (width 0.4) (layer "B.Cu") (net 20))
 (segment (start 166.873589 117.3075) (end 168.147684 116.033405) (width 0.4) (layer "B.Cu") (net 20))
 (segment (start 162.837684 99.107684) (end 162.837684 97.0875) (width 0.8) (layer "B.Cu") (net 20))
 (segment (start 162.957684 99.227684) (end 162.957684 96.9675) (width 0.8) (layer "B.Cu") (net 20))
 (segment (start 158.915685 119.0575) (end 160.665685 117.3075) (width 0.4) (layer "B.Cu") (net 20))
 (segment (start 163.24 99.51) (end 162.837684 99.107684) (width 0.8) (layer "B.Cu") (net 20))
 (segment (start 150.977684 119.0575) (end 158.915685 119.0575) (width 0.4) (layer "B.Cu") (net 20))
 (segment (start 149.967684 118.0475) (end 150.977684 119.0575) (width 0.4) (layer "B.Cu") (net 20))
 (segment (start 157.347684 111.3475) (end 159.397684 111.3475) (width 0.4) (layer "F.Cu") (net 1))
 (segment (start 159.397684 111.3475) (end 160.327684 110.4175) (width 0.4) (layer "F.Cu") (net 1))
 (via (at 160.327684 110.4175) (size 1.6256) (drill 0.8128) (layers "F.Cu" "B.Cu") (free yes) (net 1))
 (segment (start 158.2775 110.4175) (end 148.257684 100.397684) (width 0.4) (layer "B.Cu") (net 1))
 (segment (start 160.327684 110.4175) (end 158.2775 110.4175) (width 0.4) (layer "B.Cu") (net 1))
 (segment (start 148.257684 100.397684) (end 148.257684 95.4675) (width 0.4) (layer "B.Cu") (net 1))
 (segment (start 164.870184 114.96) (end 166.39 114.96) (width 0.4) (layer "B.Cu") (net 1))
 (segment (start 160.327684 110.4175) (end 164.870184 114.96) (width 0.4) (layer "B.Cu") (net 1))
 (segment (start 146.28 123.591) (end 150.695184 123.591) (width 0.4) (layer "F.Cu") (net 19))
 (segment (start 157.28 123.471) (end 153.475184 123.471) (width 0.4) (layer "F.Cu") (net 21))
 (segment (start 153.437684 123.5085) (end 156.177684 123.5085) (width 0.4) (layer "F.Cu") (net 21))
 (segment (start 153.475184 123.471) (end 153.437684 123.5085) (width 0.4) (layer "F.Cu") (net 21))
 (segment (start 148.524884 117.462299) (end 148.524884 119.7393) (width 0.4) (layer "F.Cu") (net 25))
 (segment (start 148.524884 119.7393) (end 147.975184 120.289) (width 0.4) (layer "F.Cu") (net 25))
 (segment (start 147.975184 120.289) (end 146.28 120.289) (width 0.4) (layer "F.Cu") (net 25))
 (segment (start 152.397684 116.4275) (end 149.559683 116.4275) (width 0.4) (layer "F.Cu") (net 25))
 (segment (start 149.559683 116.4275) (end 148.524884 117.462299) (width 0.4) (layer "F.Cu") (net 25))
 (segment (start 145.678144 103.4075) (end 140.317684 103.4075) (width 0.8) (layer "F.Cu") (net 4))
 (segment (start 153.726284 96.90936) (end 154.758144 95.8775) (width 0.8) (layer "F.Cu") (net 4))
 (segment (start 140.317684 103.4075) (end 138.237684 101.3275) (width 0.8) (layer "F.Cu") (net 4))
 (segment (start 138.237684 101.3275) (end 138.237684 100.9175) (width 0.8) (layer "F.Cu") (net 4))
 (segment (start 138.247684 100.9075) (end 138.247684 99.0675) (width 0.8) (layer "F.Cu") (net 4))
 (segment (start 139.860484 97.4547) (end 138.247684 99.0675) (width 0.8) (layer "F.Cu") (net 4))
 (segment (start 152.082284 97.4547) (end 139.860484 97.4547) (width 0.8) (layer "F.Cu") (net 4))
 (segment (start 153.726284 99.0987) (end 152.082284 97.4547) (width 0.8) (layer "F.Cu") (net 4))
 (segment (start 138.237684 100.9175) (end 138.247684 100.9075) (width 0.8) (layer "F.Cu") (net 4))
 (segment (start 144.412684 105.4925) (end 144.412684 104.67296) (width 0.8) (layer "F.Cu") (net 4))
 (segment (start 145.678144 103.4075) (end 146.43 104.159356) (width 0.8) (layer "F.Cu") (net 4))
 (segment (start 153.726284 99.0987) (end 153.726284 96.90936) (width 0.8) (layer "F.Cu") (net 4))
 (segment (start 144.412684 104.67296) (end 145.678144 103.4075) (width 0.8) (layer "F.Cu") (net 4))
 (via (at 141.217684 117.9375) (size 1.6256) (drill 0.8128) (layers "F.Cu" "B.Cu") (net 4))
 (via (at 138.247684 99.0675) (size 1.6256) (drill 0.8128) (layers "F.Cu" "B.Cu") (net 4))
 (segment (start 138.247684 99.092316) (end 145 105.844632) (width 0.8) (layer "B.Cu") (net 4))
 (segment (start 138.247684 95.4775) (end 138.257684 95.4675) (width 0.8) (layer "B.Cu") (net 4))
 (segment (start 145 105.844632) (end 145 114.155184) (width 0.8) (layer "B.Cu") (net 4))
 (segment (start 141.217684 117.9375) (end 138.857684 117.9375) (width 0.8) (layer "B.Cu") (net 4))
 (segment (start 138.857684 117.9375) (end 138.797684 117.8775) (width 0.8) (layer "B.Cu") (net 4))
 (segment (start 138.247684 99.0675) (end 138.247684 99.092316) (width 0.8) (layer "B.Cu") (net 4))
 (segment (start 138.247684 99.0675) (end 138.247684 96.46) (width 0.8) (layer "B.Cu") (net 4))
 (segment (start 145 114.155184) (end 141.217684 117.9375) (width 0.8) (layer "B.Cu") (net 4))
 (segment (start 138.247684 96.46) (end 138.247684 95.4775) (width 0.8) (layer "B.Cu") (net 4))
 (segment (start 152.397684 113.8875) (end 150.9075 113.8875) (width 0.4) (layer "F.Cu") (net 6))
 (segment (start 150.1325 113.1125) (end 149.362684 113.1125) (width 0.4) (layer "F.Cu") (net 6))
 (segment (start 150.9075 113.8875) (end 150.1325 113.1125) (width 0.4) (layer "F.Cu") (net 6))
 (segment (start 150.9075 111.3475) (end 150.1325 110.5725) (width 0.4) (layer "F.Cu") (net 8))
 (segment (start 150.1325 110.5725) (end 149.362684 110.5725) (width 0.4) (layer "F.Cu") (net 8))
 (segment (start 152.397684 111.3475) (end 150.9075 111.3475) (width 0.4) (layer "F.Cu") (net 8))
 (segment (start 150.1325 111.8425) (end 149.362684 111.8425) (width 0.4) (layer "F.Cu") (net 7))
 (segment (start 150.9075 112.6175) (end 150.1325 111.8425) (width 0.4) (layer "F.Cu") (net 7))
 (segment (start 152.397684 112.6175) (end 150.9075 112.6175) (width 0.4) (layer "F.Cu") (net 7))
 (segment (start 152.397684 115.1575) (end 150.137684 115.1575) (width 0.4) (layer "F.Cu") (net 5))
 (segment (start 150.137684 115.1575) (end 149.362684 114.3825) (width 0.4) (layer "F.Cu") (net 5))
 (segment (start 160.297684 112.6175) (end 160.327684 112.6475) (width 0.4) (layer "F.Cu") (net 24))
 (segment (start 157.347684 112.6175) (end 160.297684 112.6175) (width 0.4) (layer "F.Cu") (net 24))
 (via (at 160.327684 112.6475) (size 1.6256) (drill 0.8128) (layers "F.Cu" "B.Cu") (free yes) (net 24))
 (segment (start 145.757684 100.477684) (end 145.757684 95.4675) (width 0.4) (layer "B.Cu") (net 24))
 (segment (start 157.9275 112.6475) (end 145.757684 100.477684) (width 0.4) (layer "B.Cu") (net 24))
 (segment (start 160.327684 112.6475) (end 157.9275 112.6475) (width 0.4) (layer "B.Cu") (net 24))
 (segment (start 157.347684 113.8875) (end 157.647683 114.187499) (width 0.4) (layer "F.Cu") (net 23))
 (segment (start 161.087683 114.187499) (end 161.437684 114.5375) (width 0.4) (layer "F.Cu") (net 23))
 (segment (start 157.647683 114.187499) (end 161.087683 114.187499) (width 0.4) (layer "F.Cu") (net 23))
 (via (at 161.437684 114.5375) (size 1.6256) (drill 0.8128) (layers "F.Cu" "B.Cu") (free yes) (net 23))
 (segment (start 156.8275 114.5375) (end 143.257684 100.967684) (width 0.4) (layer "B.Cu") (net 23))
 (segment (start 161.437684 114.5375) (end 156.8275 114.5375) (width 0.4) (layer "B.Cu") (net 23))
 (segment (start 143.257684 100.967684) (end 143.257684 95.4675) (width 0.4) (layer "B.Cu") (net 23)))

